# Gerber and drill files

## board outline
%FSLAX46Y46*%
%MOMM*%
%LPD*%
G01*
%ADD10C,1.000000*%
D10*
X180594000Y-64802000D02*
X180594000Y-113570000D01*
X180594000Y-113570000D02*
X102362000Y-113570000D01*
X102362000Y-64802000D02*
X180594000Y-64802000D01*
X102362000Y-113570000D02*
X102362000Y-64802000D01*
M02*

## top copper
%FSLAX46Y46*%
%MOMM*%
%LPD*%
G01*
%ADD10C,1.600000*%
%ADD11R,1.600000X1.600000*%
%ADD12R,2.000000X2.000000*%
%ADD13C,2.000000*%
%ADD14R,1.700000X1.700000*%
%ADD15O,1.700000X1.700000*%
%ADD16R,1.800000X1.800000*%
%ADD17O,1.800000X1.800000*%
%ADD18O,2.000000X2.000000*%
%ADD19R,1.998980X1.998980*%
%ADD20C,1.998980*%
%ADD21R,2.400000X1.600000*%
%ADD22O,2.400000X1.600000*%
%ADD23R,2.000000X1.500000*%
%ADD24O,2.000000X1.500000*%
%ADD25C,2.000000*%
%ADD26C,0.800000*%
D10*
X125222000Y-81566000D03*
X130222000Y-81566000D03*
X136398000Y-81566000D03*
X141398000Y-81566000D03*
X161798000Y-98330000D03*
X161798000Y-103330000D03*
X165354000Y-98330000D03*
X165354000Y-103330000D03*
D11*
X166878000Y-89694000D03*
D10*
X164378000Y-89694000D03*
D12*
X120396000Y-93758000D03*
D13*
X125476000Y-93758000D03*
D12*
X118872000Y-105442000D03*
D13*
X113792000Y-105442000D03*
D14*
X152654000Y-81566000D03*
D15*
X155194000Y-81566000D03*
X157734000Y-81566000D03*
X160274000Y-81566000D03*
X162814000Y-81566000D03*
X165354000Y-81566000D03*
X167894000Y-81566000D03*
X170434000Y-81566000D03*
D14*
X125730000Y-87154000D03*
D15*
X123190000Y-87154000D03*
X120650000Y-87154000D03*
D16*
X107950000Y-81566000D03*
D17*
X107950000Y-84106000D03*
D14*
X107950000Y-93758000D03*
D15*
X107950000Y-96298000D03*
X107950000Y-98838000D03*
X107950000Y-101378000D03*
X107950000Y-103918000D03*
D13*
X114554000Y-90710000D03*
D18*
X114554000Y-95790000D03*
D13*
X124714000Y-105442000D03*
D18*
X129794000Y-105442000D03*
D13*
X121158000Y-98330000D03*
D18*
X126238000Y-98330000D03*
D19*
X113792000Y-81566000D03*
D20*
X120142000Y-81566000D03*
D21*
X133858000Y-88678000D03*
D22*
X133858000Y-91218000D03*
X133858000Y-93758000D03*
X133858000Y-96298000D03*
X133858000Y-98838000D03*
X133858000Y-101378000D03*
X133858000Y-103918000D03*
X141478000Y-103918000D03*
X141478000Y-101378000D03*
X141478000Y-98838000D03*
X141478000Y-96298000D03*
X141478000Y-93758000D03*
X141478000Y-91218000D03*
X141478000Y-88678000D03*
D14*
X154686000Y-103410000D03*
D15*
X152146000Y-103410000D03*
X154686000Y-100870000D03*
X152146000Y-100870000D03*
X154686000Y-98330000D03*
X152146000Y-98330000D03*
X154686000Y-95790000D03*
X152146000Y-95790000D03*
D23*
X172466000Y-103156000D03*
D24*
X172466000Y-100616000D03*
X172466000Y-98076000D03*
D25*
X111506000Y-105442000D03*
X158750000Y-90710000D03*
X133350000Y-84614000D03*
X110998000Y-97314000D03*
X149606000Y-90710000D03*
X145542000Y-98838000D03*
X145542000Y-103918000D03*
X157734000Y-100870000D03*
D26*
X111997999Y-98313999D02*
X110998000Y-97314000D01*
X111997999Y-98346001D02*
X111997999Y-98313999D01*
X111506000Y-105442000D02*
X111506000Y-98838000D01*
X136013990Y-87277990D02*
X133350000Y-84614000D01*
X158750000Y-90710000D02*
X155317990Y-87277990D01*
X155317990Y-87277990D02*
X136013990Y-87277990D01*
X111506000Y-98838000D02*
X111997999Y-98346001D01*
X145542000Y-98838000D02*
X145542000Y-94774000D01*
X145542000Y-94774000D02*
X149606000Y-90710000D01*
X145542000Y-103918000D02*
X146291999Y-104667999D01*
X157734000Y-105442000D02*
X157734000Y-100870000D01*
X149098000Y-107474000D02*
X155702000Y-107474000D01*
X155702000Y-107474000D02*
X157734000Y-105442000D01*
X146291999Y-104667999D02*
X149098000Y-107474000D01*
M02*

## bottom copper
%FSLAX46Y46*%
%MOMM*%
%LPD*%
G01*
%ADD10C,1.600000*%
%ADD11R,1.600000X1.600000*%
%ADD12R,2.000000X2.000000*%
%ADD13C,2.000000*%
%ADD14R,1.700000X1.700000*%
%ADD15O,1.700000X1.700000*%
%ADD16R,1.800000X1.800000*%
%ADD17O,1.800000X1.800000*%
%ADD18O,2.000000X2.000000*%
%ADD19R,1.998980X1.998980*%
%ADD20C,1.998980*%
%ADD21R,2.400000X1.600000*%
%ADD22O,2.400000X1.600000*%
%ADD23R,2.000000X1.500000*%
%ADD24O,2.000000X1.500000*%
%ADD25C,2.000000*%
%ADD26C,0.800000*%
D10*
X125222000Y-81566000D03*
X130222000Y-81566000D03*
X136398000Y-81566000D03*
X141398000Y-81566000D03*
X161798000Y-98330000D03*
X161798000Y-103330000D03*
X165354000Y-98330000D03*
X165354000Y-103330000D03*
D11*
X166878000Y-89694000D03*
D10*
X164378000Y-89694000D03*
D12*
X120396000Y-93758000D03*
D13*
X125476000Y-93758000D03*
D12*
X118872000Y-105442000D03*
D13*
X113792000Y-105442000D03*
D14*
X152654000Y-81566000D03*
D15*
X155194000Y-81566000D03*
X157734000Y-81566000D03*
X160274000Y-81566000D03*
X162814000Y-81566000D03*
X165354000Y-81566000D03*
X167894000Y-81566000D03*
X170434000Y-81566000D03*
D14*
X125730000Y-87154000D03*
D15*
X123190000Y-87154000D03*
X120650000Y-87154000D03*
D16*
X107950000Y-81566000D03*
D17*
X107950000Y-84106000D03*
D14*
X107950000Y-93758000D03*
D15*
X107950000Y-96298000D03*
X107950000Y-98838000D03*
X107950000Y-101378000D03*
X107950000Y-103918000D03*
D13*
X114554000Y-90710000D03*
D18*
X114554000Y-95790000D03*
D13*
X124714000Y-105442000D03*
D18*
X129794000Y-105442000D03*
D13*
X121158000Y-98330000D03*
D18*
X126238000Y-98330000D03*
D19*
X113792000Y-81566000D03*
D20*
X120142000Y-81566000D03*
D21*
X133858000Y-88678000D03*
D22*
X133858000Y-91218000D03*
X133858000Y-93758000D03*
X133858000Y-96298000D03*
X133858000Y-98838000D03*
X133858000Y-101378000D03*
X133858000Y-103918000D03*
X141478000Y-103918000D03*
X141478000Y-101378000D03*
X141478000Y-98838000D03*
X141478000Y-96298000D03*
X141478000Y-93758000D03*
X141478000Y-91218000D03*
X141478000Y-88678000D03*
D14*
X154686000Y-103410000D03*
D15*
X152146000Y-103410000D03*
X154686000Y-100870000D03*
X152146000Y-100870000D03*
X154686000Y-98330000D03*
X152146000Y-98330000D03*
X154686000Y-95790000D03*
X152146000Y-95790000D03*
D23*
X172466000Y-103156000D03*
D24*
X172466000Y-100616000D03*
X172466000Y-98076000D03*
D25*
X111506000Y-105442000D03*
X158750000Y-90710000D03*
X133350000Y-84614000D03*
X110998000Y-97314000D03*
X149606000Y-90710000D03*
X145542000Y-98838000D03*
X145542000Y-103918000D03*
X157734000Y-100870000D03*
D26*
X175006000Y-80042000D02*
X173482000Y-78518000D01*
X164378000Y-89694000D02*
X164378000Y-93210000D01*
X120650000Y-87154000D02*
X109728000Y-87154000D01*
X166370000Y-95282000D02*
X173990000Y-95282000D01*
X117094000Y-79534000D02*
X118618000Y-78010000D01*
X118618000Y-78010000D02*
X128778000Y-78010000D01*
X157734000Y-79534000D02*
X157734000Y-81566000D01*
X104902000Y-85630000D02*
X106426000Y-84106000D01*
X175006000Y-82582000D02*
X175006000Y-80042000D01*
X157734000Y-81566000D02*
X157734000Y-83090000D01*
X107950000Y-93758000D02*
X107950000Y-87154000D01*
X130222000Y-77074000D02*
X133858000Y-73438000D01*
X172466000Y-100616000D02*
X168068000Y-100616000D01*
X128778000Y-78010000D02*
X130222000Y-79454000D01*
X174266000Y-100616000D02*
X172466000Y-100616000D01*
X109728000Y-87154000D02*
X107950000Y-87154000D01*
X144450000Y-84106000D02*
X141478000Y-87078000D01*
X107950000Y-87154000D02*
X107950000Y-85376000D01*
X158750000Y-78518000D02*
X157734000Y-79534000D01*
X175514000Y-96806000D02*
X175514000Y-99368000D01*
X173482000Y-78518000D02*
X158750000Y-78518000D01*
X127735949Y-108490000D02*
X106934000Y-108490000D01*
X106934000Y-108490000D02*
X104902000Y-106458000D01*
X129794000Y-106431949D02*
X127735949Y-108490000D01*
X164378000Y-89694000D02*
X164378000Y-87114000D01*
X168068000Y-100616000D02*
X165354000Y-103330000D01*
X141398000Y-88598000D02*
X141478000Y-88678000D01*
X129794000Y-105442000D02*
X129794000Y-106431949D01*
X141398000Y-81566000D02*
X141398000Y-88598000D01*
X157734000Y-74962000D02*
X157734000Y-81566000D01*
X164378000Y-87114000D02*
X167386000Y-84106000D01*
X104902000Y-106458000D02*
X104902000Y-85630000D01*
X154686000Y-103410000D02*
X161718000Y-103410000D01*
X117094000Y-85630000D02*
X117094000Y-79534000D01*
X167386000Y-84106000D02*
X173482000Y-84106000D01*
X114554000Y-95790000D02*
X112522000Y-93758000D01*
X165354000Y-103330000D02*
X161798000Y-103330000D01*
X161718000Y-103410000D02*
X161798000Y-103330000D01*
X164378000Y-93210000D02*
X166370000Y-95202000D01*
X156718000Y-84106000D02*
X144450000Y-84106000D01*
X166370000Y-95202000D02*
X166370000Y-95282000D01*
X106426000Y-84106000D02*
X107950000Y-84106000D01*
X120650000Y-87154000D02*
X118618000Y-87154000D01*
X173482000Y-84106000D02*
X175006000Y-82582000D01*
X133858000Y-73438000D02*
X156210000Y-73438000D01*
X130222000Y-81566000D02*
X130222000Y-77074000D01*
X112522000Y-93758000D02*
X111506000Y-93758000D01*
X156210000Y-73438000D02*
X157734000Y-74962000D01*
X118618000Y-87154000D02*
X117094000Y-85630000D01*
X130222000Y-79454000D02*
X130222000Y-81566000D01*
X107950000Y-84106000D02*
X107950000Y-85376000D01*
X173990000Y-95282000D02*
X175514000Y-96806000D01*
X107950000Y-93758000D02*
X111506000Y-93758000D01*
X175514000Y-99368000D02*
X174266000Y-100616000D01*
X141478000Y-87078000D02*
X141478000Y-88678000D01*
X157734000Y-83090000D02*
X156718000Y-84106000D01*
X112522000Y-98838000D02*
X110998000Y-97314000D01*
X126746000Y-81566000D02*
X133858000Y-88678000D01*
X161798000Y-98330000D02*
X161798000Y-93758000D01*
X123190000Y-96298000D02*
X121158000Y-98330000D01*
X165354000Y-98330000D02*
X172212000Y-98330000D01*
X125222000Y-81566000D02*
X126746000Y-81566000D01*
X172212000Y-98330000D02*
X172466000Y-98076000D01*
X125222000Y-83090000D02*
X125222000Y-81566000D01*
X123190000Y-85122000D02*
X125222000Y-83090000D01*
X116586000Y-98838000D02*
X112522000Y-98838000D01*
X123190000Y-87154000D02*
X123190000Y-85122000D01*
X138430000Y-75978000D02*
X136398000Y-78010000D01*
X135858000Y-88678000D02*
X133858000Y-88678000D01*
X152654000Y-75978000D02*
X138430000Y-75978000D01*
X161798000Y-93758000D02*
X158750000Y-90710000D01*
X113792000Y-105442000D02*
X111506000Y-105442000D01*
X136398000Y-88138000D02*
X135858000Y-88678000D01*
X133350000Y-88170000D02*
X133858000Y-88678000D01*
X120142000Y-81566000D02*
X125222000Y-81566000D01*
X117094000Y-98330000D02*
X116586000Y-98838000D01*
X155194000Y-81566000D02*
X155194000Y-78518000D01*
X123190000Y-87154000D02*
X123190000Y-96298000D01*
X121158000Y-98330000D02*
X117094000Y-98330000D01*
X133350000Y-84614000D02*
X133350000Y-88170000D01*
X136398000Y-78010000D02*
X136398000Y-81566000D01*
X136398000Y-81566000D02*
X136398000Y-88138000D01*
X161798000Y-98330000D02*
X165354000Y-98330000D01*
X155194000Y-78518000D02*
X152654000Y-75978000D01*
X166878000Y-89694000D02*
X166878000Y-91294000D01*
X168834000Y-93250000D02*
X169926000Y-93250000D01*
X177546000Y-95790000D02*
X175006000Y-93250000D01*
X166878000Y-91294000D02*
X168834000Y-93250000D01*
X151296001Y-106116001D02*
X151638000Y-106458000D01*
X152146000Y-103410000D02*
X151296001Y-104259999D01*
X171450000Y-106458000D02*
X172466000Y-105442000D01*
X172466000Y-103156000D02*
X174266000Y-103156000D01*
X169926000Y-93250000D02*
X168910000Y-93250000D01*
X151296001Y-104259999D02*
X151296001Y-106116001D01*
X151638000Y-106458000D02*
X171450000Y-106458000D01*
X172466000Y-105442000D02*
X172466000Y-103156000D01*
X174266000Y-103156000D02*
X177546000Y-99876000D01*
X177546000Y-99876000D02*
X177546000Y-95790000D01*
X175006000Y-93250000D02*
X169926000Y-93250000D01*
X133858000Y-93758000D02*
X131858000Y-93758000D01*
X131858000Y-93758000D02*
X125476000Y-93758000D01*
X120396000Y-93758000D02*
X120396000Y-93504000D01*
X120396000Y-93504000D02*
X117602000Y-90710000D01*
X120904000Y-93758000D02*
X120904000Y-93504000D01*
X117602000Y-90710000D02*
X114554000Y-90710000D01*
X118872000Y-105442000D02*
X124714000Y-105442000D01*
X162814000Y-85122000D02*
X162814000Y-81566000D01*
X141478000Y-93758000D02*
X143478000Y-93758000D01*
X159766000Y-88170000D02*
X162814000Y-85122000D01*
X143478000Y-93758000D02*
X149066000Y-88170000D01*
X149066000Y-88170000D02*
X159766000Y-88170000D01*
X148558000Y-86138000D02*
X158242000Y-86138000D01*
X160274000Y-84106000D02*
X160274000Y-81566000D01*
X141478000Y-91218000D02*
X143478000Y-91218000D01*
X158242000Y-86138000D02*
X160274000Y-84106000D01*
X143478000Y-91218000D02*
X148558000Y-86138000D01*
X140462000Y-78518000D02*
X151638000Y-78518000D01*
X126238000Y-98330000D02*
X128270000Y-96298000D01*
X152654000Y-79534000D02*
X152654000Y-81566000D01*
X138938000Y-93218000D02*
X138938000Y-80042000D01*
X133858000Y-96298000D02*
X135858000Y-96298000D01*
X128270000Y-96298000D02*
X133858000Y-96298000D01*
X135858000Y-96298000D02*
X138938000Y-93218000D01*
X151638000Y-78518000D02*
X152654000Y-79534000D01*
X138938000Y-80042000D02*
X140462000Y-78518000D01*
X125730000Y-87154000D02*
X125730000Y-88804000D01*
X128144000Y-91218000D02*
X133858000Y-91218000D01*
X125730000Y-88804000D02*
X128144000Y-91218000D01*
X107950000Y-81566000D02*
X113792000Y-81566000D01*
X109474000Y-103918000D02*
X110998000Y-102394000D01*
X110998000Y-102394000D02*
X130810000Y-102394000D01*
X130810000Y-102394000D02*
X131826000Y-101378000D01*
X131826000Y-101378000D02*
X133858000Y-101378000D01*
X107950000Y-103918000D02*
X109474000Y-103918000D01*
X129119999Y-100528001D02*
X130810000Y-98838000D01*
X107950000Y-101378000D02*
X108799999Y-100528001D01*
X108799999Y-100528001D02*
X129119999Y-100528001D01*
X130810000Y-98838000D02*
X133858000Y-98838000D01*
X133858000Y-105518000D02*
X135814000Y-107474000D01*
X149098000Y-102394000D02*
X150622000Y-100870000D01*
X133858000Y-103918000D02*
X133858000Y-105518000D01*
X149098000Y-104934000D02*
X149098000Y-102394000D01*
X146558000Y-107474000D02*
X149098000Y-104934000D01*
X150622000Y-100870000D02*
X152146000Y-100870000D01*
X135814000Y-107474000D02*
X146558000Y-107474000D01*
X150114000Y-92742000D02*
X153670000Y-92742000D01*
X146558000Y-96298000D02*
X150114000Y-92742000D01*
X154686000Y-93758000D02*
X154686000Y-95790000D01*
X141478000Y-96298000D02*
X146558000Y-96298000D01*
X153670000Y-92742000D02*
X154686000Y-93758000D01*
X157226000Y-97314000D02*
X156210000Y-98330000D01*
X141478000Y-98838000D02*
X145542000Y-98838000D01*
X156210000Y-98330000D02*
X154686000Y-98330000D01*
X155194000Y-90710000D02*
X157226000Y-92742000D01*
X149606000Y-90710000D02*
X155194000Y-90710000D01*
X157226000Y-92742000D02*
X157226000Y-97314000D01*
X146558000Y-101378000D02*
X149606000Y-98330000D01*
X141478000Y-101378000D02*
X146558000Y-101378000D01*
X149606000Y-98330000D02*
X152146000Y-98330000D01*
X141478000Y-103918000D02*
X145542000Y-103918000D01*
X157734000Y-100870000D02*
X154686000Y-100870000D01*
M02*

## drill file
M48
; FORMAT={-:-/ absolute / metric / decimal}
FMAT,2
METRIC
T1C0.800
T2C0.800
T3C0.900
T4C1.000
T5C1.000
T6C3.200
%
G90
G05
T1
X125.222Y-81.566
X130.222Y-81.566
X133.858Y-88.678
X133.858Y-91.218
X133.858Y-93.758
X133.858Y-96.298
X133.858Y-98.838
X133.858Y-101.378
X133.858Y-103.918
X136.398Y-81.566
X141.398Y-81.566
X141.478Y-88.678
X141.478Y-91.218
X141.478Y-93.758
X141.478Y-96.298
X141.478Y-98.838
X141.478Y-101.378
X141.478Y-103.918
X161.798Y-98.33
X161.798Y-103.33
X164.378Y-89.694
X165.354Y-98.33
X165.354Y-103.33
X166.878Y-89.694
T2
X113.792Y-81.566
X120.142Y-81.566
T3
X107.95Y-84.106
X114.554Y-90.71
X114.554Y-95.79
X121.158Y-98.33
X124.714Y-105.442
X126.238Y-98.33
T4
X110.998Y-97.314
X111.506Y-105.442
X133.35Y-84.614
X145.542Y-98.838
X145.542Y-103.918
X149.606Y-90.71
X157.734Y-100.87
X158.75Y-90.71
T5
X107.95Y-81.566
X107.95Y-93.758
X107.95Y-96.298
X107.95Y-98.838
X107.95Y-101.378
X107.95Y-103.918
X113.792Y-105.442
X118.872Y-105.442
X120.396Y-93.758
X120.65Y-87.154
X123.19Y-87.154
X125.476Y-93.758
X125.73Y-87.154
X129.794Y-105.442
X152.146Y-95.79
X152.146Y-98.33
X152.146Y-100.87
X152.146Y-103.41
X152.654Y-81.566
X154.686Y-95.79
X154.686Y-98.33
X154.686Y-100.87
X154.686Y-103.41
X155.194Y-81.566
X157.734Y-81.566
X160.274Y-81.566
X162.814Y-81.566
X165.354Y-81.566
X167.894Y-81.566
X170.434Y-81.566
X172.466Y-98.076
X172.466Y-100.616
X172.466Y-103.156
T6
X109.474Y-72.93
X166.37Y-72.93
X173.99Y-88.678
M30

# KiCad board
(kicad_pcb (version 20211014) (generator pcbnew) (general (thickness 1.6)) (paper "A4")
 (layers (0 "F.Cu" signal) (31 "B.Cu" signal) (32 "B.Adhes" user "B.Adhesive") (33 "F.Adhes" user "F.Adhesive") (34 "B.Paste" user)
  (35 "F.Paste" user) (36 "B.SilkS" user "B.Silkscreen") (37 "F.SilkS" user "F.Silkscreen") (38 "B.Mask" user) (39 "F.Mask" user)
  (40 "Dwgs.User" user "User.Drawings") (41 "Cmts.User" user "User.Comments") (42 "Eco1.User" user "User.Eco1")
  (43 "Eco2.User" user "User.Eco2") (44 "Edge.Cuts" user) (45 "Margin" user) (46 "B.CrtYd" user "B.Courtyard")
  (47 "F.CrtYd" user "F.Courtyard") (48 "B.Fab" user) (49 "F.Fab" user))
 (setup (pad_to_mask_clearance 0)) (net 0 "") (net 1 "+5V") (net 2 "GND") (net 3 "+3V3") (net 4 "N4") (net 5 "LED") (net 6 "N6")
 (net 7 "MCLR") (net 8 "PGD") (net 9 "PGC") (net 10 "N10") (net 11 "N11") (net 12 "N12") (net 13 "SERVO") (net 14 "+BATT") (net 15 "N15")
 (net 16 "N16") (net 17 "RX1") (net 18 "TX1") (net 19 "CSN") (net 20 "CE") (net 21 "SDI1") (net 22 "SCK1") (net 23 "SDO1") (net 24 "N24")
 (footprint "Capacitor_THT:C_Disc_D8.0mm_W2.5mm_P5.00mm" (layer "F.Cu") (at 125.222 81.566)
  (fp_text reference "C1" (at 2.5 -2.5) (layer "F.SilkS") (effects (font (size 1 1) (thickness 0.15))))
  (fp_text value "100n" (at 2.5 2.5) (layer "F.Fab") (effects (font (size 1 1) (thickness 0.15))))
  (pad "1" thru_hole circle locked (at 0 0) (size 1.6 1.6) (drill 0.8) (layers *.Cu *.Mask) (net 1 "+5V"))
  (pad "2" thru_hole circle locked (at 5 0) (size 1.6 1.6) (drill 0.8) (layers *.Cu *.Mask) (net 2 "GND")))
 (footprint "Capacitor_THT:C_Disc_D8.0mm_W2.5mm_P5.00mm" (layer "F.Cu") (at 136.398 81.566)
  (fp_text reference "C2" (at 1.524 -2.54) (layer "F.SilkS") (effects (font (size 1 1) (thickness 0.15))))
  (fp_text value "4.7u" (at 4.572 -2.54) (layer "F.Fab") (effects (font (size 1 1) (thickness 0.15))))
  (pad "1" thru_hole circle locked (at 0 0) (size 1.6 1.6) (drill 0.8) (layers *.Cu *.Mask) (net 1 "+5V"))
  (pad "2" thru_hole circle locked (at 5 0) (size 1.6 1.6) (drill 0.8) (layers *.Cu *.Mask) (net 2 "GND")))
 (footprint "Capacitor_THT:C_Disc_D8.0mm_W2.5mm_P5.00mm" (layer "F.Cu") (at 161.798 98.33 -90)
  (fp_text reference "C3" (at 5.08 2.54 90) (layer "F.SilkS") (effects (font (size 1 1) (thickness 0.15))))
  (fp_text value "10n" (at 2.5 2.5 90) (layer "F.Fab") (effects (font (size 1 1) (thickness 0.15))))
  (pad "1" thru_hole circle locked (at 0 0 270) (size 1.6 1.6) (drill 0.8) (layers *.Cu *.Mask) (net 1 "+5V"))
  (pad "2" thru_hole circle locked (at 5 0 270) (size 1.6 1.6) (drill 0.8) (layers *.Cu *.Mask) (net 2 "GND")))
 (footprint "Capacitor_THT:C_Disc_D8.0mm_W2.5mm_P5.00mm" (layer "F.Cu") (at 165.354 98.33 -90)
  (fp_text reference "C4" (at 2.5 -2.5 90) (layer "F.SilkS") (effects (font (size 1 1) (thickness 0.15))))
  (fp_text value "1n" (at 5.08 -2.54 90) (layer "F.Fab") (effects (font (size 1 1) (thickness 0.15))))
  (pad "1" thru_hole circle locked (at 0 0 270) (size 1.6 1.6) (drill 0.8) (layers *.Cu *.Mask) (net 1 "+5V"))
  (pad "2" thru_hole circle locked (at 5 0 270) (size 1.6 1.6) (drill 0.8) (layers *.Cu *.Mask) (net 2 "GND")))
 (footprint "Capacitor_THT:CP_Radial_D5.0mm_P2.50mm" (layer "F.Cu") (at 166.878 89.694 180)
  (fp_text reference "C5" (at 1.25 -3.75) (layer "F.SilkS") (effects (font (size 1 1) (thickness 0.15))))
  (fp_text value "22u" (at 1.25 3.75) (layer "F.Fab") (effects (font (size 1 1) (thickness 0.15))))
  (pad "1" thru_hole rect locked (at 0 0 180) (size 1.6 1.6) (drill 0.8) (layers *.Cu *.Mask) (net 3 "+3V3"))
  (pad "2" thru_hole circle locked (at 2.5 0 180) (size 1.6 1.6) (drill 0.8) (layers *.Cu *.Mask) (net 2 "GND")))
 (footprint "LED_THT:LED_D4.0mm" (layer "F.Cu") (at 121.666 93.758)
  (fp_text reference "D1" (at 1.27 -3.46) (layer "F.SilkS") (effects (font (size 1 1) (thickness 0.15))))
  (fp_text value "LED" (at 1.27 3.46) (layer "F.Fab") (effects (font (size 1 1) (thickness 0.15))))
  (pad "1" thru_hole rect locked (at -1.27 0) (size 2 2) (drill 1) (layers *.Cu *.Mask) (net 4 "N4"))
  (pad "2" thru_hole circle locked (at 3.81 0) (size 2 2) (drill 1) (layers *.Cu *.Mask) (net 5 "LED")))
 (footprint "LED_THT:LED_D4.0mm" (layer "F.Cu") (at 117.602 105.442 180)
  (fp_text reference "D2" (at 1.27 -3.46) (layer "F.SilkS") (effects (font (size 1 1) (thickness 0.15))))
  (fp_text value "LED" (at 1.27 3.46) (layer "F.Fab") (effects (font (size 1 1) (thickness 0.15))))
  (pad "1" thru_hole rect locked (at -1.27 0 180) (size 2 2) (drill 1) (layers *.Cu *.Mask) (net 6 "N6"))
  (pad "2" thru_hole circle locked (at 3.81 0 180) (size 2 2) (drill 1) (layers *.Cu *.Mask) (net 1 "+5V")))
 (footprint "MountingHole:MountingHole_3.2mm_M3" (layer "F.Cu") (at 166.37 72.93)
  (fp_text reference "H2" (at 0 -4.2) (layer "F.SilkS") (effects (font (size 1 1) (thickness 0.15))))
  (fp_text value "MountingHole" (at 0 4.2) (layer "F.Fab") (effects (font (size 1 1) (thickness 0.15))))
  (pad "" np_thru_hole circle locked (at 0 0) (size 3.2 3.2) (drill 3.2) (layers *.Cu *.Mask)))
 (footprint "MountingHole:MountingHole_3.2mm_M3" (layer "F.Cu") (at 173.99 88.678)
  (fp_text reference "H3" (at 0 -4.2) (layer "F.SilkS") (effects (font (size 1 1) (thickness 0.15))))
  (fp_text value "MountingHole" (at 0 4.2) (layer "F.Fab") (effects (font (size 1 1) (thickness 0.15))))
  (pad "" np_thru_hole circle locked (at 0 0) (size 3.2 3.2) (drill 3.2) (layers *.Cu *.Mask)))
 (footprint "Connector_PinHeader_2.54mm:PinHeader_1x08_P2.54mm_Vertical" (layer "F.Cu") (at 152.654 81.566 90)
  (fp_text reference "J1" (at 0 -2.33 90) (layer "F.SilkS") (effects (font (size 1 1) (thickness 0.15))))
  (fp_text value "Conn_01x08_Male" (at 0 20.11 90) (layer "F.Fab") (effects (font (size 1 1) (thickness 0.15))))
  (pad "1" thru_hole rect locked (at 0 0 90) (size 1.7 1.7) (drill 1) (layers *.Cu *.Mask) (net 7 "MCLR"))
  (pad "2" thru_hole oval locked (at 0 2.54 90) (size 1.7 1.7) (drill 1) (layers *.Cu *.Mask) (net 1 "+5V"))
  (pad "3" thru_hole oval locked (at 0 5.08 90) (size 1.7 1.7) (drill 1) (layers *.Cu *.Mask) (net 2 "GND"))
  (pad "4" thru_hole oval locked (at 0 7.62 90) (size 1.7 1.7) (drill 1) (layers *.Cu *.Mask) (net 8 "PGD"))
  (pad "5" thru_hole oval locked (at 0 10.16 90) (size 1.7 1.7) (drill 1) (layers *.Cu *.Mask) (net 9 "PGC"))
  (pad "6" thru_hole oval locked (at 0 12.7 90) (size 1.7 1.7) (drill 1) (layers *.Cu *.Mask) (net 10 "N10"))
  (pad "7" thru_hole oval locked (at 0 15.24 90) (size 1.7 1.7) (drill 1) (layers *.Cu *.Mask) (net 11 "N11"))
  (pad "8" thru_hole oval locked (at 0 17.78 90) (size 1.7 1.7) (drill 1) (layers *.Cu *.Mask) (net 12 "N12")))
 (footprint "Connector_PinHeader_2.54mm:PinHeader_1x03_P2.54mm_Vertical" (layer "F.Cu") (at 125.73 87.154 -90)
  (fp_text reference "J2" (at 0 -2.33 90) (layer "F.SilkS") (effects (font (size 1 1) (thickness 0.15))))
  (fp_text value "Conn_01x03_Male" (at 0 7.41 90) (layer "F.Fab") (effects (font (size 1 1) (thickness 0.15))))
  (pad "1" thru_hole rect locked (at 0 0 270) (size 1.7 1.7) (drill 1) (layers *.Cu *.Mask) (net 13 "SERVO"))
  (pad "2" thru_hole oval locked (at 0 2.54 270) (size 1.7 1.7) (drill 1) (layers *.Cu *.Mask) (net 1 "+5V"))
  (pad "3" thru_hole oval locked (at 0 5.08 270) (size 1.7 1.7) (drill 1) (layers *.Cu *.Mask) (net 2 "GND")))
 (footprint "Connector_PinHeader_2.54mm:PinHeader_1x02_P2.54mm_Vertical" (layer "F.Cu") (at 107.95 81.566)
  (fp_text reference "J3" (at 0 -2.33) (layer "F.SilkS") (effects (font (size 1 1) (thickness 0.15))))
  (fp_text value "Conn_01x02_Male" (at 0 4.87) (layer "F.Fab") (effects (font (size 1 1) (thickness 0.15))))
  (pad "1" thru_hole rect locked (at 0 0) (size 1.8 1.8) (drill 1) (layers *.Cu *.Mask) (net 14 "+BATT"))
  (pad "2" thru_hole oval locked (at 0 2.54) (size 1.8 1.8) (drill 0.9) (layers *.Cu *.Mask) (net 2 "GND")))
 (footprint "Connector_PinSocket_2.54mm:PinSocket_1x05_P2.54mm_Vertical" (layer "F.Cu") (at 107.95 93.758)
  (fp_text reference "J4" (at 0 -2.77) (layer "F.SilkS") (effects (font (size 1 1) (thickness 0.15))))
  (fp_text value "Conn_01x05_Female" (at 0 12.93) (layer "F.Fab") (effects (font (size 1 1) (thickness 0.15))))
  (pad "1" thru_hole rect locked (at 0 0) (size 1.7 1.7) (drill 1) (layers *.Cu *.Mask) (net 2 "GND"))
  (pad "2" thru_hole oval locked (at 0 2.54) (size 1.7 1.7) (drill 1) (layers *.Cu *.Mask) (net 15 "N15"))
  (pad "3" thru_hole oval locked (at 0 5.08) (size 1.7 1.7) (drill 1) (layers *.Cu *.Mask) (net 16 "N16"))
  (pad "4" thru_hole oval locked (at 0 7.62) (size 1.7 1.7) (drill 1) (layers *.Cu *.Mask) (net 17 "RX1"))
  (pad "5" thru_hole oval locked (at 0 10.16) (size 1.7 1.7) (drill 1) (layers *.Cu *.Mask) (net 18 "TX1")))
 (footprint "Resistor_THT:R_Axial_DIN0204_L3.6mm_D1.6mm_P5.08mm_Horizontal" (layer "F.Cu") (at 114.554 90.71 -90)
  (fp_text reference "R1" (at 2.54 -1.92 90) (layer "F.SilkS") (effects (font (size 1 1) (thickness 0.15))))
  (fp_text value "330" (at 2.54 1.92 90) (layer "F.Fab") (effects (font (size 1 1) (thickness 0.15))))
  (pad "1" thru_hole circle locked (at 0 0 270) (size 2 2) (drill 0.9) (layers *.Cu *.Mask) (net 4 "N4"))
  (pad "2" thru_hole oval locked (at 5.08 0 270) (size 2 2) (drill 0.9) (layers *.Cu *.Mask) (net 2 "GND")))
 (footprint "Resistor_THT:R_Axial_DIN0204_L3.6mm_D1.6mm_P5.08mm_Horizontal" (layer "F.Cu") (at 124.714 105.442)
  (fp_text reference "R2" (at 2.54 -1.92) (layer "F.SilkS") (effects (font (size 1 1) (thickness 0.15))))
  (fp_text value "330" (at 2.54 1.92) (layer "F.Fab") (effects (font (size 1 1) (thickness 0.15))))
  (pad "1" thru_hole circle locked (at 0 0) (size 2 2) (drill 0.9) (layers *.Cu *.Mask) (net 6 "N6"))
  (pad "2" thru_hole oval locked (at 5.08 0) (size 2 2) (drill 1) (layers *.Cu *.Mask) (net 2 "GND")))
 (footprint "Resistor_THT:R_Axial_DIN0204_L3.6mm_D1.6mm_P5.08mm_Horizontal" (layer "F.Cu") (at 121.158 98.33)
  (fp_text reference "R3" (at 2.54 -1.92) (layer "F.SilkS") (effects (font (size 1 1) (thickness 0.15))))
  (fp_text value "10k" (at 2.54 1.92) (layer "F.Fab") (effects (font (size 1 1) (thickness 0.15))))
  (pad "1" thru_hole circle locked (at 0 0) (size 2 2) (drill 0.9) (layers *.Cu *.Mask) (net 1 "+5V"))
  (pad "2" thru_hole oval locked (at 5.08 0) (size 2 2) (drill 0.9) (layers *.Cu *.Mask) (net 7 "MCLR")))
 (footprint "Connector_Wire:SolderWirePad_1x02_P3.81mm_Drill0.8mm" (layer "F.Cu") (at 115.062 81.566)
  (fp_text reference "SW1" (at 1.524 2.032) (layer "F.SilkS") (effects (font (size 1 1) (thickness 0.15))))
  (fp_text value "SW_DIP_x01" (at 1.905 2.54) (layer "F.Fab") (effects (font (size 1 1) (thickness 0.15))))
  (pad "1" thru_hole rect locked (at -1.27 0) (size 1.99898 1.99898) (drill 0.8001) (layers *.Cu *.Mask) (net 14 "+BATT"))
  (pad "2" thru_hole circle locked (at 5.08 0) (size 1.99898 1.99898) (drill 0.8001) (layers *.Cu *.Mask) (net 1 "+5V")))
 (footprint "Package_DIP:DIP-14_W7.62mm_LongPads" (layer "F.Cu") (at 133.858 88.678)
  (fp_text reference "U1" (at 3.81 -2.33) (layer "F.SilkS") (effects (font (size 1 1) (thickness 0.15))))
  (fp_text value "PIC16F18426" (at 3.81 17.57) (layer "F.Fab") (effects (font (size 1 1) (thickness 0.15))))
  (pad "1" thru_hole rect locked (at 0 0) (size 2.4 1.6) (drill 0.8) (layers *.Cu *.Mask) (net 1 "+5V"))
  (pad "2" thru_hole oval locked (at 0 2.54) (size 2.4 1.6) (drill 0.8) (layers *.Cu *.Mask) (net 13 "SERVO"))
  (pad "3" thru_hole oval locked (at 0 5.08) (size 2.4 1.6) (drill 0.8) (layers *.Cu *.Mask) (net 5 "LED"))
  (pad "4" thru_hole oval locked (at 0 7.62) (size 2.4 1.6) (drill 0.8) (layers *.Cu *.Mask) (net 7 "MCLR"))
  (pad "5" thru_hole oval locked (at 0 10.16) (size 2.4 1.6) (drill 0.8) (layers *.Cu *.Mask) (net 17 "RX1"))
  (pad "6" thru_hole oval locked (at 0 12.7) (size 2.4 1.6) (drill 0.8) (layers *.Cu *.Mask) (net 18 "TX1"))
  (pad "7" thru_hole oval locked (at 0 15.24) (size 2.4 1.6) (drill 0.8) (layers *.Cu *.Mask) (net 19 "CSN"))
  (pad "8" thru_hole oval locked (at 7.62 15.24) (size 2.4 1.6) (drill 0.8) (layers *.Cu *.Mask) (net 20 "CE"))
  (pad "9" thru_hole oval locked (at 7.62 12.7) (size 2.4 1.6) (drill 0.8) (layers *.Cu *.Mask) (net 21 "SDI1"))
  (pad "10" thru_hole oval locked (at 7.62 10.16) (size 2.4 1.6) (drill 0.8) (layers *.Cu *.Mask) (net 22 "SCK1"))
  (pad "11" thru_hole oval locked (at 7.62 7.62) (size 2.4 1.6) (drill 0.8) (layers *.Cu *.Mask) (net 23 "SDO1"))
  (pad "12" thru_hole oval locked (at 7.62 5.08) (size 2.4 1.6) (drill 0.8) (layers *.Cu *.Mask) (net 9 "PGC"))
  (pad "13" thru_hole oval locked (at 7.62 2.54) (size 2.4 1.6) (drill 0.8) (layers *.Cu *.Mask) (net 8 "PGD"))
  (pad "14" thru_hole oval locked (at 7.62 0) (size 2.4 1.6) (drill 0.8) (layers *.Cu *.Mask) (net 2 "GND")))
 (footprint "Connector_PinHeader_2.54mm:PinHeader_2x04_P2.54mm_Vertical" (layer "F.Cu") (at 154.686 103.41 180)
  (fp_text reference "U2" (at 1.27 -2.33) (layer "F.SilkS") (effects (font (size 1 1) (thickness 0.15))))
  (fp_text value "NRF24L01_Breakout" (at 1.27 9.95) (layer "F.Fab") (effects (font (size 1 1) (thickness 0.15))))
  (pad "1" thru_hole rect locked (at 0 0 180) (size 1.7 1.7) (drill 1) (layers *.Cu *.Mask) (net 2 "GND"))
  (pad "2" thru_hole oval locked (at 2.54 0 180) (size 1.7 1.7) (drill 1) (layers *.Cu *.Mask) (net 3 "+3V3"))
  (pad "3" thru_hole oval locked (at 0 2.54 180) (size 1.7 1.7) (drill 1) (layers *.Cu *.Mask) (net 20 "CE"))
  (pad "4" thru_hole oval locked (at 2.54 2.54 180) (size 1.7 1.7) (drill 1) (layers *.Cu *.Mask) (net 19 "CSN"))
  (pad "5" thru_hole oval locked (at 0 5.08 180) (size 1.7 1.7) (drill 1) (layers *.Cu *.Mask) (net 22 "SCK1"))
  (pad "6" thru_hole oval locked (at 2.54 5.08 180) (size 1.7 1.7) (drill 1) (layers *.Cu *.Mask) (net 21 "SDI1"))
  (pad "7" thru_hole oval locked (at 0 7.62 180) (size 1.7 1.7) (drill 1) (layers *.Cu *.Mask) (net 23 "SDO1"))
  (pad "8" thru_hole oval locked (at 2.54 7.62 180) (size 1.7 1.7) (drill 1) (layers *.Cu *.Mask) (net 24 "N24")))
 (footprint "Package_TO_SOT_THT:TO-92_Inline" (layer "F.Cu") (at 172.466 101.886 90)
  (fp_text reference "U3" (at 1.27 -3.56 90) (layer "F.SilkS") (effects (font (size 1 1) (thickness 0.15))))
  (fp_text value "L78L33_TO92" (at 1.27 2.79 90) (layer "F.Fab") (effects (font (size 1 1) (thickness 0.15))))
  (pad "1" thru_hole rect locked (at -1.27 0 90) (size 1.5 2) (drill 1) (layers *.Cu *.Mask) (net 3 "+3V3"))
  (pad "2" thru_hole oval locked (at 1.27 0 90) (size 1.5 2) (drill 1) (layers *.Cu *.Mask) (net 2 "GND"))
  (pad "3" thru_hole oval locked (at 3.81 0 90) (size 1.5 2) (drill 1) (layers *.Cu *.Mask) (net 1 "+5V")))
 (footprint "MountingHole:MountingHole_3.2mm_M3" (layer "F.Cu") (at 109.474 72.93)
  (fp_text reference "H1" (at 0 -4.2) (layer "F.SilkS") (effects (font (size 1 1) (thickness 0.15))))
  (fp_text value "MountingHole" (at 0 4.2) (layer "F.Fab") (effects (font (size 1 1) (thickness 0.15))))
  (pad "" np_thru_hole circle locked (at 0 0) (size 3.2 3.2) (drill 3.2) (layers *.Cu *.Mask)))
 (gr_line (start 180.594 64.802) (end 180.594 113.57) (layer "Edge.Cuts") (width 1))
 (gr_line (start 180.594 113.57) (end 102.362 113.57) (layer "Edge.Cuts") (width 1))
 (gr_line (start 102.362 64.802) (end 180.594 64.802) (layer "Edge.Cuts") (width 1))
 (gr_line (start 102.362 113.57) (end 102.362 64.802) (layer "Edge.Cuts") (width 1))
 (segment (start 175.006 80.042) (end 173.482 78.518) (width 0.8) (layer "B.Cu") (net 2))
 (segment (start 164.378 89.694) (end 164.378 93.21) (width 0.8) (layer "B.Cu") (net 2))
 (segment (start 120.65 87.154) (end 109.728 87.154) (width 0.8) (layer "B.Cu") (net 2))
 (segment (start 166.37 95.282) (end 173.99 95.282) (width 0.8) (layer "B.Cu") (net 2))
 (segment (start 117.094 79.534) (end 118.618 78.01) (width 0.8) (layer "B.Cu") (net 2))
 (segment (start 118.618 78.01) (end 128.778 78.01) (width 0.8) (layer "B.Cu") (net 2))
 (segment (start 157.734 79.534) (end 157.734 81.566) (width 0.8) (layer "B.Cu") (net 2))
 (segment (start 104.902 85.63) (end 106.426 84.106) (width 0.8) (layer "B.Cu") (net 2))
 (segment (start 175.006 82.582) (end 175.006 80.042) (width 0.8) (layer "B.Cu") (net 2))
 (segment (start 157.734 81.566) (end 157.734 83.09) (width 0.8) (layer "B.Cu") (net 2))
 (segment (start 107.95 93.758) (end 107.95 87.154) (width 0.8) (layer "B.Cu") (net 2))
 (segment (start 130.222 77.074) (end 133.858 73.438) (width 0.8) (layer "B.Cu") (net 2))
 (segment (start 172.466 100.616) (end 168.068 100.616) (width 0.8) (layer "B.Cu") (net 2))
 (segment (start 128.778 78.01) (end 130.222 79.454) (width 0.8) (layer "B.Cu") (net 2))
 (segment (start 174.266 100.616) (end 172.466 100.616) (width 0.8) (layer "B.Cu") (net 2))
 (segment (start 109.728 87.154) (end 107.95 87.154) (width 0.8) (layer "B.Cu") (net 2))
 (segment (start 144.45 84.106) (end 141.478 87.078) (width 0.8) (layer "B.Cu") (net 2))
 (segment (start 107.95 87.154) (end 107.95 85.376) (width 0.8) (layer "B.Cu") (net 2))
 (segment (start 158.75 78.518) (end 157.734 79.534) (width 0.8) (layer "B.Cu") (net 2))
 (segment (start 175.514 96.806) (end 175.514 99.368) (width 0.8) (layer "B.Cu") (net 2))
 (segment (start 173.482 78.518) (end 158.75 78.518) (width 0.8) (layer "B.Cu") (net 2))
 (segment (start 127.735949 108.49) (end 106.934 108.49) (width 0.8) (layer "B.Cu") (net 2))
 (segment (start 106.934 108.49) (end 104.902 106.458) (width 0.8) (layer "B.Cu") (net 2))
 (segment (start 129.794 106.431949) (end 127.735949 108.49) (width 0.8) (layer "B.Cu") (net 2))
 (segment (start 164.378 89.694) (end 164.378 87.114) (width 0.8) (layer "B.Cu") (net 2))
 (segment (start 168.068 100.616) (end 165.354 103.33) (width 0.8) (layer "B.Cu") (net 2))
 (segment (start 141.398 88.598) (end 141.478 88.678) (width 0.8) (layer "B.Cu") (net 2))
 (segment (start 129.794 105.442) (end 129.794 106.431949) (width 0.8) (layer "B.Cu") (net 2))
 (segment (start 141.398 81.566) (end 141.398 88.598) (width 0.8) (layer "B.Cu") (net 2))
 (segment (start 157.734 74.962) (end 157.734 81.566) (width 0.8) (layer "B.Cu") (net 2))
 (segment (start 164.378 87.114) (end 167.386 84.106) (width 0.8) (layer "B.Cu") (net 2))
 (segment (start 104.902 106.458) (end 104.902 85.63) (width 0.8) (layer "B.Cu") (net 2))
 (segment (start 154.686 103.41) (end 161.718 103.41) (width 0.8) (layer "B.Cu") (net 2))
 (segment (start 117.094 85.63) (end 117.094 79.534) (width 0.8) (layer "B.Cu") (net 2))
 (segment (start 167.386 84.106) (end 173.482 84.106) (width 0.8) (layer "B.Cu") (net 2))
 (segment (start 114.554 95.79) (end 112.522 93.758) (width 0.8) (layer "B.Cu") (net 2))
 (segment (start 165.354 103.33) (end 161.798 103.33) (width 0.8) (layer "B.Cu") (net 2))
 (segment (start 161.718 103.41) (end 161.798 103.33) (width 0.8) (layer "B.Cu") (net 2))
 (segment (start 164.378 93.21) (end 166.37 95.202) (width 0.8) (layer "B.Cu") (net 2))
 (segment (start 156.718 84.106) (end 144.45 84.106) (width 0.8) (layer "B.Cu") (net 2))
 (segment (start 166.37 95.202) (end 166.37 95.282) (width 0.8) (layer "B.Cu") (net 2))
 (segment (start 106.426 84.106) (end 107.95 84.106) (width 0.8) (layer "B.Cu") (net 2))
 (segment (start 120.65 87.154) (end 118.618 87.154) (width 0.8) (layer "B.Cu") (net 2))
 (segment (start 173.482 84.106) (end 175.006 82.582) (width 0.8) (layer "B.Cu") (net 2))
 (segment (start 133.858 73.438) (end 156.21 73.438) (width 0.8) (layer "B.Cu") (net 2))
 (segment (start 130.222 81.566) (end 130.222 77.074) (width 0.8) (layer "B.Cu") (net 2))
 (segment (start 112.522 93.758) (end 111.506 93.758) (width 0.8) (layer "B.Cu") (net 2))
 (segment (start 156.21 73.438) (end 157.734 74.962) (width 0.8) (layer "B.Cu") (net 2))
 (segment (start 118.618 87.154) (end 117.094 85.63) (width 0.8) (layer "B.Cu") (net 2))
 (segment (start 130.222 79.454) (end 130.222 81.566) (width 0.8) (layer "B.Cu") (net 2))
 (segment (start 107.95 84.106) (end 107.95 85.376) (width 0.8) (layer "B.Cu") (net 2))
 (segment (start 173.99 95.282) (end 175.514 96.806) (width 0.8) (layer "B.Cu") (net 2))
 (segment (start 107.95 93.758) (end 111.506 93.758) (width 0.8) (layer "B.Cu") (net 2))
 (segment (start 175.514 99.368) (end 174.266 100.616) (width 0.8) (layer "B.Cu") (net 2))
 (segment (start 141.478 87.078) (end 141.478 88.678) (width 0.8) (layer "B.Cu") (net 2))
 (segment (start 157.734 83.09) (end 156.718 84.106) (width 0.8) (layer "B.Cu") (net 2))
 (segment (start 111.997999 98.313999) (end 110.998 97.314) (width 0.8) (layer "F.Cu") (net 1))
 (segment (start 111.997999 98.346001) (end 111.997999 98.313999) (width 0.8) (layer "F.Cu") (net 1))
 (segment (start 111.506 105.442) (end 111.506 98.838) (width 0.8) (layer "F.Cu") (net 1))
 (segment (start 136.01399 87.27799) (end 133.35 84.614) (width 0.8) (layer "F.Cu") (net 1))
 (segment (start 158.75 90.71) (end 155.31799 87.27799) (width 0.8) (layer "F.Cu") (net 1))
 (segment (start 155.31799 87.27799) (end 136.01399 87.27799) (width 0.8) (layer "F.Cu") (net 1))
 (segment (start 111.506 98.838) (end 111.997999 98.346001) (width 0.8) (layer "F.Cu") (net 1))
 (via (at 111.506 105.442) (size 2) (drill 1) (layers "F.Cu" "B.Cu") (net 1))
 (via (at 158.75 90.71) (size 2) (drill 1) (layers "F.Cu" "B.Cu") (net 1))
 (via (at 133.35 84.614) (size 2) (drill 1) (layers "F.Cu" "B.Cu") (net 1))
 (via (at 110.998 97.314) (size 2) (drill 1) (layers "F.Cu" "B.Cu") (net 1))
 (segment (start 112.522 98.838) (end 110.998 97.314) (width 0.8) (layer "B.Cu") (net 1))
 (segment (start 126.746 81.566) (end 133.858 88.678) (width 0.8) (layer "B.Cu") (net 1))
 (segment (start 161.798 98.33) (end 161.798 93.758) (width 0.8) (layer "B.Cu") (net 1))
 (segment (start 123.19 96.298) (end 121.158 98.33) (width 0.8) (layer "B.Cu") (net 1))
 (segment (start 165.354 98.33) (end 172.212 98.33) (width 0.8) (layer "B.Cu") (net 1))
 (segment (start 125.222 81.566) (end 126.746 81.566) (width 0.8) (layer "B.Cu") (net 1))
 (segment (start 172.212 98.33) (end 172.466 98.076) (width 0.8) (layer "B.Cu") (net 1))
 (segment (start 125.222 83.09) (end 125.222 81.566) (width 0.8) (layer "B.Cu") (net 1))
 (segment (start 123.19 85.122) (end 125.222 83.09) (width 0.8) (layer "B.Cu") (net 1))
 (segment (start 116.586 98.838) (end 112.522 98.838) (width 0.8) (layer "B.Cu") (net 1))
 (segment (start 123.19 87.154) (end 123.19 85.122) (width 0.8) (layer "B.Cu") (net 1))
 (segment (start 138.43 75.978) (end 136.398 78.01) (width 0.8) (layer "B.Cu") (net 1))
 (segment (start 135.858 88.678) (end 133.858 88.678) (width 0.8) (layer "B.Cu") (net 1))
 (segment (start 152.654 75.978) (end 138.43 75.978) (width 0.8) (layer "B.Cu") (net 1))
 (segment (start 161.798 93.758) (end 158.75 90.71) (width 0.8) (layer "B.Cu") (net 1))
 (segment (start 113.792 105.442) (end 111.506 105.442) (width 0.8) (layer "B.Cu") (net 1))
 (segment (start 136.398 88.138) (end 135.858 88.678) (width 0.8) (layer "B.Cu") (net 1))
 (segment (start 133.35 88.17) (end 133.858 88.678) (width 0.8) (layer "B.Cu") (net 1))
 (segment (start 120.142 81.566) (end 125.222 81.566) (width 0.8) (layer "B.Cu") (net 1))
 (segment (start 117.094 98.33) (end 116.586 98.838) (width 0.8) (layer "B.Cu") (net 1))
 (segment (start 155.194 81.566) (end 155.194 78.518) (width 0.8) (layer "B.Cu") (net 1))
 (segment (start 123.19 87.154) (end 123.19 96.298) (width 0.8) (layer "B.Cu") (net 1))
 (segment (start 121.158 98.33) (end 117.094 98.33) (width 0.8) (layer "B.Cu") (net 1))
 (segment (start 133.35 84.614) (end 133.35 88.17) (width 0.8) (layer "B.Cu") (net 1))
 (segment (start 136.398 78.01) (end 136.398 81.566) (width 0.8) (layer "B.Cu") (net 1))
 (segment (start 136.398 81.566) (end 136.398 88.138) (width 0.8) (layer "B.Cu") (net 1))
 (segment (start 161.798 98.33) (end 165.354 98.33) (width 0.8) (layer "B.Cu") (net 1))
 (segment (start 155.194 78.518) (end 152.654 75.978) (width 0.8) (layer "B.Cu") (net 1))
 (segment (start 166.878 89.694) (end 166.878 91.294) (width 0.8) (layer "B.Cu") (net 3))
 (segment (start 168.834 93.25) (end 169.926 93.25) (width 0.8) (layer "B.Cu") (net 3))
 (segment (start 177.546 95.79) (end 175.006 93.25) (width 0.8) (layer "B.Cu") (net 3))
 (segment (start 166.878 91.294) (end 168.834 93.25) (width 0.8) (layer "B.Cu") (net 3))
 (segment (start 151.296001 106.116001) (end 151.638 106.458) (width 0.8) (layer "B.Cu") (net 3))
 (segment (start 152.146 103.41) (end 151.296001 104.259999) (width 0.8) (layer "B.Cu") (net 3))
 (segment (start 171.45 106.458) (end 172.466 105.442) (width 0.8) (layer "B.Cu") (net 3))
 (segment (start 172.466 103.156) (end 174.266 103.156) (width 0.8) (layer "B.Cu") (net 3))
 (segment (start 169.926 93.25) (end 168.91 93.25) (width 0.8) (layer "B.Cu") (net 3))
 (segment (start 151.296001 104.259999) (end 151.296001 106.116001) (width 0.8) (layer "B.Cu") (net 3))
 (segment (start 151.638 106.458) (end 171.45 106.458) (width 0.8) (layer "B.Cu") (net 3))
 (segment (start 172.466 105.442) (end 172.466 103.156) (width 0.8) (layer "B.Cu") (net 3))
 (segment (start 174.266 103.156) (end 177.546 99.876) (width 0.8) (layer "B.Cu") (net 3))
 (segment (start 177.546 99.876) (end 177.546 95.79) (width 0.8) (layer "B.Cu") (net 3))
 (segment (start 175.006 93.25) (end 169.926 93.25) (width 0.8) (layer "B.Cu") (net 3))
 (segment (start 133.858 93.758) (end 131.858 93.758) (width 0.8) (layer "B.Cu") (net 5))
 (segment (start 131.858 93.758) (end 125.476 93.758) (width 0.8) (layer "B.Cu") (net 5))
 (segment (start 120.396 93.758) (end 120.396 93.504) (width 0.8) (layer "B.Cu") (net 4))
 (segment (start 120.396 93.504) (end 117.602 90.71) (width 0.8) (layer "B.Cu") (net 4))
 (segment (start 120.904 93.758) (end 120.904 93.504) (width 0.8) (layer "B.Cu") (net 4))
 (segment (start 117.602 90.71) (end 114.554 90.71) (width 0.8) (layer "B.Cu") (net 4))
 (segment (start 118.872 105.442) (end 124.714 105.442) (width 0.8) (layer "B.Cu") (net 6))
 (segment (start 162.814 85.122) (end 162.814 81.566) (width 0.8) (layer "B.Cu") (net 9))
 (segment (start 141.478 93.758) (end 143.478 93.758) (width 0.8) (layer "B.Cu") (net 9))
 (segment (start 159.766 88.17) (end 162.814 85.122) (width 0.8) (layer "B.Cu") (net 9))
 (segment (start 143.478 93.758) (end 149.066 88.17) (width 0.8) (layer "B.Cu") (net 9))
 (segment (start 149.066 88.17) (end 159.766 88.17) (width 0.8) (layer "B.Cu") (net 9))
 (segment (start 148.558 86.138) (end 158.242 86.138) (width 0.8) (layer "B.Cu") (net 8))
 (segment (start 160.274 84.106) (end 160.274 81.566) (width 0.8) (layer "B.Cu") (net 8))
 (segment (start 141.478 91.218) (end 143.478 91.218) (width 0.8) (layer "B.Cu") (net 8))
 (segment (start 158.242 86.138) (end 160.274 84.106) (width 0.8) (layer "B.Cu") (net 8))
 (segment (start 143.478 91.218) (end 148.558 86.138) (width 0.8) (layer "B.Cu") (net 8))
 (segment (start 140.462 78.518) (end 151.638 78.518) (width 0.8) (layer "B.Cu") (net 7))
 (segment (start 126.238 98.33) (end 128.27 96.298) (width 0.8) (layer "B.Cu") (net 7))
 (segment (start 152.654 79.534) (end 152.654 81.566) (width 0.8) (layer "B.Cu") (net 7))
 (segment (start 138.938 93.218) (end 138.938 80.042) (width 0.8) (layer "B.Cu") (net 7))
 (segment (start 133.858 96.298) (end 135.858 96.298) (width 0.8) (layer "B.Cu") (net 7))
 (segment (start 128.27 96.298) (end 133.858 96.298) (width 0.8) (layer "B.Cu") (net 7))
 (segment (start 135.858 96.298) (end 138.938 93.218) (width 0.8) (layer "B.Cu") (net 7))
 (segment (start 151.638 78.518) (end 152.654 79.534) (width 0.8) (layer "B.Cu") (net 7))
 (segment (start 138.938 80.042) (end 140.462 78.518) (width 0.8) (layer "B.Cu") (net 7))
 (segment (start 125.73 87.154) (end 125.73 88.804) (width 0.8) (layer "B.Cu") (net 13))
 (segment (start 128.144 91.218) (end 133.858 91.218) (width 0.8) (layer "B.Cu") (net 13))
 (segment (start 125.73 88.804) (end 128.144 91.218) (width 0.8) (layer "B.Cu") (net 13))
 (segment (start 107.95 81.566) (end 113.792 81.566) (width 0.8) (layer "B.Cu") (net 14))
 (segment (start 109.474 103.918) (end 110.998 102.394) (width 0.8) (layer "B.Cu") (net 18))
 (segment (start 110.998 102.394) (end 130.81 102.394) (width 0.8) (layer "B.Cu") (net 18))
 (segment (start 130.81 102.394) (end 131.826 101.378) (width 0.8) (layer "B.Cu") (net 18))
 (segment (start 131.826 101.378) (end 133.858 101.378) (width 0.8) (layer "B.Cu") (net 18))
 (segment (start 107.95 103.918) (end 109.474 103.918) (width 0.8) (layer "B.Cu") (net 18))
 (segment (start 129.119999 100.528001) (end 130.81 98.838) (width 0.8) (layer "B.Cu") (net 17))
 (segment (start 107.95 101.378) (end 108.799999 100.528001) (width 0.8) (layer "B.Cu") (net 17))
 (segment (start 108.799999 100.528001) (end 129.119999 100.528001) (width 0.8) (layer "B.Cu") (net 17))
 (segment (start 130.81 98.838) (end 133.858 98.838) (width 0.8) (layer "B.Cu") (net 17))
 (segment (start 133.858 105.518) (end 135.814 107.474) (width 0.8) (layer "B.Cu") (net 19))
 (segment (start 149.098 102.394) (end 150.622 100.87) (width 0.8) (layer "B.Cu") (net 19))
 (segment (start 133.858 103.918) (end 133.858 105.518) (width 0.8) (layer "B.Cu") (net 19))
 (segment (start 149.098 104.934) (end 149.098 102.394) (width 0.8) (layer "B.Cu") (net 19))
 (segment (start 146.558 107.474) (end 149.098 104.934) (width 0.8) (layer "B.Cu") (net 19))
 (segment (start 150.622 100.87) (end 152.146 100.87) (width 0.8) (layer "B.Cu") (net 19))
 (segment (start 135.814 107.474) (end 146.558 107.474) (width 0.8) (layer "B.Cu") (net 19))
 (segment (start 150.114 92.742) (end 153.67 92.742) (width 0.8) (layer "B.Cu") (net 23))
 (segment (start 146.558 96.298) (end 150.114 92.742) (width 0.8) (layer "B.Cu") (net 23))
 (segment (start 154.686 93.758) (end 154.686 95.79) (width 0.8) (layer "B.Cu") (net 23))
 (segment (start 141.478 96.298) (end 146.558 96.298) (width 0.8) (layer "B.Cu") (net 23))
 (segment (start 153.67 92.742) (end 154.686 93.758) (width 0.8) (layer "B.Cu") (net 23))
 (segment (start 145.542 98.838) (end 145.542 94.774) (width 0.8) (layer "F.Cu") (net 22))
 (segment (start 145.542 94.774) (end 149.606 90.71) (width 0.8) (layer "F.Cu") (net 22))
 (via (at 149.606 90.71) (size 2) (drill 1) (layers "F.Cu" "B.Cu") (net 22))
 (via (at 145.542 98.838) (size 2) (drill 1) (layers "F.Cu" "B.Cu") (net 22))
 (segment (start 157.226 97.314) (end 156.21 98.33) (width 0.8) (layer "B.Cu") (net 22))
 (segment (start 141.478 98.838) (end 145.542 98.838) (width 0.8) (layer "B.Cu") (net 22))
 (segment (start 156.21 98.33) (end 154.686 98.33) (width 0.8) (layer "B.Cu") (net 22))
 (segment (start 155.194 90.71) (end 157.226 92.742) (width 0.8) (layer "B.Cu") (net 22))
 (segment (start 149.606 90.71) (end 155.194 90.71) (width 0.8) (layer "B.Cu") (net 22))
 (segment (start 157.226 92.742) (end 157.226 97.314) (width 0.8) (layer "B.Cu") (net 22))
 (segment (start 146.558 101.378) (end 149.606 98.33) (width 0.8) (layer "B.Cu") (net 21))
 (segment (start 141.478 101.378) (end 146.558 101.378) (width 0.8) (layer "B.Cu") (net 21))
 (segment (start 149.606 98.33) (end 152.146 98.33) (width 0.8) (layer "B.Cu") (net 21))
 (segment (start 145.542 103.918) (end 146.291999 104.667999) (width 0.8) (layer "F.Cu") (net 20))
 (segment (start 157.734 105.442) (end 157.734 100.87) (width 0.8) (layer "F.Cu") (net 20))
 (segment (start 149.098 107.474) (end 155.702 107.474) (width 0.8) (layer "F.Cu") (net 20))
 (segment (start 155.702 107.474) (end 157.734 105.442) (width 0.8) (layer "F.Cu") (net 20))
 (segment (start 146.291999 104.667999) (end 149.098 107.474) (width 0.8) (layer "F.Cu") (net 20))
 (via (at 145.542 103.918) (size 2) (drill 1) (layers "F.Cu" "B.Cu") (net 20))
 (via (at 157.734 100.87) (size 2) (drill 1) (layers "F.Cu" "B.Cu") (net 20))
 (segment (start 141.478 103.918) (end 145.542 103.918) (width 0.8) (layer "B.Cu") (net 20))
 (segment (start 157.734 100.87) (end 154.686 100.87) (width 0.8) (layer "B.Cu") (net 20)))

